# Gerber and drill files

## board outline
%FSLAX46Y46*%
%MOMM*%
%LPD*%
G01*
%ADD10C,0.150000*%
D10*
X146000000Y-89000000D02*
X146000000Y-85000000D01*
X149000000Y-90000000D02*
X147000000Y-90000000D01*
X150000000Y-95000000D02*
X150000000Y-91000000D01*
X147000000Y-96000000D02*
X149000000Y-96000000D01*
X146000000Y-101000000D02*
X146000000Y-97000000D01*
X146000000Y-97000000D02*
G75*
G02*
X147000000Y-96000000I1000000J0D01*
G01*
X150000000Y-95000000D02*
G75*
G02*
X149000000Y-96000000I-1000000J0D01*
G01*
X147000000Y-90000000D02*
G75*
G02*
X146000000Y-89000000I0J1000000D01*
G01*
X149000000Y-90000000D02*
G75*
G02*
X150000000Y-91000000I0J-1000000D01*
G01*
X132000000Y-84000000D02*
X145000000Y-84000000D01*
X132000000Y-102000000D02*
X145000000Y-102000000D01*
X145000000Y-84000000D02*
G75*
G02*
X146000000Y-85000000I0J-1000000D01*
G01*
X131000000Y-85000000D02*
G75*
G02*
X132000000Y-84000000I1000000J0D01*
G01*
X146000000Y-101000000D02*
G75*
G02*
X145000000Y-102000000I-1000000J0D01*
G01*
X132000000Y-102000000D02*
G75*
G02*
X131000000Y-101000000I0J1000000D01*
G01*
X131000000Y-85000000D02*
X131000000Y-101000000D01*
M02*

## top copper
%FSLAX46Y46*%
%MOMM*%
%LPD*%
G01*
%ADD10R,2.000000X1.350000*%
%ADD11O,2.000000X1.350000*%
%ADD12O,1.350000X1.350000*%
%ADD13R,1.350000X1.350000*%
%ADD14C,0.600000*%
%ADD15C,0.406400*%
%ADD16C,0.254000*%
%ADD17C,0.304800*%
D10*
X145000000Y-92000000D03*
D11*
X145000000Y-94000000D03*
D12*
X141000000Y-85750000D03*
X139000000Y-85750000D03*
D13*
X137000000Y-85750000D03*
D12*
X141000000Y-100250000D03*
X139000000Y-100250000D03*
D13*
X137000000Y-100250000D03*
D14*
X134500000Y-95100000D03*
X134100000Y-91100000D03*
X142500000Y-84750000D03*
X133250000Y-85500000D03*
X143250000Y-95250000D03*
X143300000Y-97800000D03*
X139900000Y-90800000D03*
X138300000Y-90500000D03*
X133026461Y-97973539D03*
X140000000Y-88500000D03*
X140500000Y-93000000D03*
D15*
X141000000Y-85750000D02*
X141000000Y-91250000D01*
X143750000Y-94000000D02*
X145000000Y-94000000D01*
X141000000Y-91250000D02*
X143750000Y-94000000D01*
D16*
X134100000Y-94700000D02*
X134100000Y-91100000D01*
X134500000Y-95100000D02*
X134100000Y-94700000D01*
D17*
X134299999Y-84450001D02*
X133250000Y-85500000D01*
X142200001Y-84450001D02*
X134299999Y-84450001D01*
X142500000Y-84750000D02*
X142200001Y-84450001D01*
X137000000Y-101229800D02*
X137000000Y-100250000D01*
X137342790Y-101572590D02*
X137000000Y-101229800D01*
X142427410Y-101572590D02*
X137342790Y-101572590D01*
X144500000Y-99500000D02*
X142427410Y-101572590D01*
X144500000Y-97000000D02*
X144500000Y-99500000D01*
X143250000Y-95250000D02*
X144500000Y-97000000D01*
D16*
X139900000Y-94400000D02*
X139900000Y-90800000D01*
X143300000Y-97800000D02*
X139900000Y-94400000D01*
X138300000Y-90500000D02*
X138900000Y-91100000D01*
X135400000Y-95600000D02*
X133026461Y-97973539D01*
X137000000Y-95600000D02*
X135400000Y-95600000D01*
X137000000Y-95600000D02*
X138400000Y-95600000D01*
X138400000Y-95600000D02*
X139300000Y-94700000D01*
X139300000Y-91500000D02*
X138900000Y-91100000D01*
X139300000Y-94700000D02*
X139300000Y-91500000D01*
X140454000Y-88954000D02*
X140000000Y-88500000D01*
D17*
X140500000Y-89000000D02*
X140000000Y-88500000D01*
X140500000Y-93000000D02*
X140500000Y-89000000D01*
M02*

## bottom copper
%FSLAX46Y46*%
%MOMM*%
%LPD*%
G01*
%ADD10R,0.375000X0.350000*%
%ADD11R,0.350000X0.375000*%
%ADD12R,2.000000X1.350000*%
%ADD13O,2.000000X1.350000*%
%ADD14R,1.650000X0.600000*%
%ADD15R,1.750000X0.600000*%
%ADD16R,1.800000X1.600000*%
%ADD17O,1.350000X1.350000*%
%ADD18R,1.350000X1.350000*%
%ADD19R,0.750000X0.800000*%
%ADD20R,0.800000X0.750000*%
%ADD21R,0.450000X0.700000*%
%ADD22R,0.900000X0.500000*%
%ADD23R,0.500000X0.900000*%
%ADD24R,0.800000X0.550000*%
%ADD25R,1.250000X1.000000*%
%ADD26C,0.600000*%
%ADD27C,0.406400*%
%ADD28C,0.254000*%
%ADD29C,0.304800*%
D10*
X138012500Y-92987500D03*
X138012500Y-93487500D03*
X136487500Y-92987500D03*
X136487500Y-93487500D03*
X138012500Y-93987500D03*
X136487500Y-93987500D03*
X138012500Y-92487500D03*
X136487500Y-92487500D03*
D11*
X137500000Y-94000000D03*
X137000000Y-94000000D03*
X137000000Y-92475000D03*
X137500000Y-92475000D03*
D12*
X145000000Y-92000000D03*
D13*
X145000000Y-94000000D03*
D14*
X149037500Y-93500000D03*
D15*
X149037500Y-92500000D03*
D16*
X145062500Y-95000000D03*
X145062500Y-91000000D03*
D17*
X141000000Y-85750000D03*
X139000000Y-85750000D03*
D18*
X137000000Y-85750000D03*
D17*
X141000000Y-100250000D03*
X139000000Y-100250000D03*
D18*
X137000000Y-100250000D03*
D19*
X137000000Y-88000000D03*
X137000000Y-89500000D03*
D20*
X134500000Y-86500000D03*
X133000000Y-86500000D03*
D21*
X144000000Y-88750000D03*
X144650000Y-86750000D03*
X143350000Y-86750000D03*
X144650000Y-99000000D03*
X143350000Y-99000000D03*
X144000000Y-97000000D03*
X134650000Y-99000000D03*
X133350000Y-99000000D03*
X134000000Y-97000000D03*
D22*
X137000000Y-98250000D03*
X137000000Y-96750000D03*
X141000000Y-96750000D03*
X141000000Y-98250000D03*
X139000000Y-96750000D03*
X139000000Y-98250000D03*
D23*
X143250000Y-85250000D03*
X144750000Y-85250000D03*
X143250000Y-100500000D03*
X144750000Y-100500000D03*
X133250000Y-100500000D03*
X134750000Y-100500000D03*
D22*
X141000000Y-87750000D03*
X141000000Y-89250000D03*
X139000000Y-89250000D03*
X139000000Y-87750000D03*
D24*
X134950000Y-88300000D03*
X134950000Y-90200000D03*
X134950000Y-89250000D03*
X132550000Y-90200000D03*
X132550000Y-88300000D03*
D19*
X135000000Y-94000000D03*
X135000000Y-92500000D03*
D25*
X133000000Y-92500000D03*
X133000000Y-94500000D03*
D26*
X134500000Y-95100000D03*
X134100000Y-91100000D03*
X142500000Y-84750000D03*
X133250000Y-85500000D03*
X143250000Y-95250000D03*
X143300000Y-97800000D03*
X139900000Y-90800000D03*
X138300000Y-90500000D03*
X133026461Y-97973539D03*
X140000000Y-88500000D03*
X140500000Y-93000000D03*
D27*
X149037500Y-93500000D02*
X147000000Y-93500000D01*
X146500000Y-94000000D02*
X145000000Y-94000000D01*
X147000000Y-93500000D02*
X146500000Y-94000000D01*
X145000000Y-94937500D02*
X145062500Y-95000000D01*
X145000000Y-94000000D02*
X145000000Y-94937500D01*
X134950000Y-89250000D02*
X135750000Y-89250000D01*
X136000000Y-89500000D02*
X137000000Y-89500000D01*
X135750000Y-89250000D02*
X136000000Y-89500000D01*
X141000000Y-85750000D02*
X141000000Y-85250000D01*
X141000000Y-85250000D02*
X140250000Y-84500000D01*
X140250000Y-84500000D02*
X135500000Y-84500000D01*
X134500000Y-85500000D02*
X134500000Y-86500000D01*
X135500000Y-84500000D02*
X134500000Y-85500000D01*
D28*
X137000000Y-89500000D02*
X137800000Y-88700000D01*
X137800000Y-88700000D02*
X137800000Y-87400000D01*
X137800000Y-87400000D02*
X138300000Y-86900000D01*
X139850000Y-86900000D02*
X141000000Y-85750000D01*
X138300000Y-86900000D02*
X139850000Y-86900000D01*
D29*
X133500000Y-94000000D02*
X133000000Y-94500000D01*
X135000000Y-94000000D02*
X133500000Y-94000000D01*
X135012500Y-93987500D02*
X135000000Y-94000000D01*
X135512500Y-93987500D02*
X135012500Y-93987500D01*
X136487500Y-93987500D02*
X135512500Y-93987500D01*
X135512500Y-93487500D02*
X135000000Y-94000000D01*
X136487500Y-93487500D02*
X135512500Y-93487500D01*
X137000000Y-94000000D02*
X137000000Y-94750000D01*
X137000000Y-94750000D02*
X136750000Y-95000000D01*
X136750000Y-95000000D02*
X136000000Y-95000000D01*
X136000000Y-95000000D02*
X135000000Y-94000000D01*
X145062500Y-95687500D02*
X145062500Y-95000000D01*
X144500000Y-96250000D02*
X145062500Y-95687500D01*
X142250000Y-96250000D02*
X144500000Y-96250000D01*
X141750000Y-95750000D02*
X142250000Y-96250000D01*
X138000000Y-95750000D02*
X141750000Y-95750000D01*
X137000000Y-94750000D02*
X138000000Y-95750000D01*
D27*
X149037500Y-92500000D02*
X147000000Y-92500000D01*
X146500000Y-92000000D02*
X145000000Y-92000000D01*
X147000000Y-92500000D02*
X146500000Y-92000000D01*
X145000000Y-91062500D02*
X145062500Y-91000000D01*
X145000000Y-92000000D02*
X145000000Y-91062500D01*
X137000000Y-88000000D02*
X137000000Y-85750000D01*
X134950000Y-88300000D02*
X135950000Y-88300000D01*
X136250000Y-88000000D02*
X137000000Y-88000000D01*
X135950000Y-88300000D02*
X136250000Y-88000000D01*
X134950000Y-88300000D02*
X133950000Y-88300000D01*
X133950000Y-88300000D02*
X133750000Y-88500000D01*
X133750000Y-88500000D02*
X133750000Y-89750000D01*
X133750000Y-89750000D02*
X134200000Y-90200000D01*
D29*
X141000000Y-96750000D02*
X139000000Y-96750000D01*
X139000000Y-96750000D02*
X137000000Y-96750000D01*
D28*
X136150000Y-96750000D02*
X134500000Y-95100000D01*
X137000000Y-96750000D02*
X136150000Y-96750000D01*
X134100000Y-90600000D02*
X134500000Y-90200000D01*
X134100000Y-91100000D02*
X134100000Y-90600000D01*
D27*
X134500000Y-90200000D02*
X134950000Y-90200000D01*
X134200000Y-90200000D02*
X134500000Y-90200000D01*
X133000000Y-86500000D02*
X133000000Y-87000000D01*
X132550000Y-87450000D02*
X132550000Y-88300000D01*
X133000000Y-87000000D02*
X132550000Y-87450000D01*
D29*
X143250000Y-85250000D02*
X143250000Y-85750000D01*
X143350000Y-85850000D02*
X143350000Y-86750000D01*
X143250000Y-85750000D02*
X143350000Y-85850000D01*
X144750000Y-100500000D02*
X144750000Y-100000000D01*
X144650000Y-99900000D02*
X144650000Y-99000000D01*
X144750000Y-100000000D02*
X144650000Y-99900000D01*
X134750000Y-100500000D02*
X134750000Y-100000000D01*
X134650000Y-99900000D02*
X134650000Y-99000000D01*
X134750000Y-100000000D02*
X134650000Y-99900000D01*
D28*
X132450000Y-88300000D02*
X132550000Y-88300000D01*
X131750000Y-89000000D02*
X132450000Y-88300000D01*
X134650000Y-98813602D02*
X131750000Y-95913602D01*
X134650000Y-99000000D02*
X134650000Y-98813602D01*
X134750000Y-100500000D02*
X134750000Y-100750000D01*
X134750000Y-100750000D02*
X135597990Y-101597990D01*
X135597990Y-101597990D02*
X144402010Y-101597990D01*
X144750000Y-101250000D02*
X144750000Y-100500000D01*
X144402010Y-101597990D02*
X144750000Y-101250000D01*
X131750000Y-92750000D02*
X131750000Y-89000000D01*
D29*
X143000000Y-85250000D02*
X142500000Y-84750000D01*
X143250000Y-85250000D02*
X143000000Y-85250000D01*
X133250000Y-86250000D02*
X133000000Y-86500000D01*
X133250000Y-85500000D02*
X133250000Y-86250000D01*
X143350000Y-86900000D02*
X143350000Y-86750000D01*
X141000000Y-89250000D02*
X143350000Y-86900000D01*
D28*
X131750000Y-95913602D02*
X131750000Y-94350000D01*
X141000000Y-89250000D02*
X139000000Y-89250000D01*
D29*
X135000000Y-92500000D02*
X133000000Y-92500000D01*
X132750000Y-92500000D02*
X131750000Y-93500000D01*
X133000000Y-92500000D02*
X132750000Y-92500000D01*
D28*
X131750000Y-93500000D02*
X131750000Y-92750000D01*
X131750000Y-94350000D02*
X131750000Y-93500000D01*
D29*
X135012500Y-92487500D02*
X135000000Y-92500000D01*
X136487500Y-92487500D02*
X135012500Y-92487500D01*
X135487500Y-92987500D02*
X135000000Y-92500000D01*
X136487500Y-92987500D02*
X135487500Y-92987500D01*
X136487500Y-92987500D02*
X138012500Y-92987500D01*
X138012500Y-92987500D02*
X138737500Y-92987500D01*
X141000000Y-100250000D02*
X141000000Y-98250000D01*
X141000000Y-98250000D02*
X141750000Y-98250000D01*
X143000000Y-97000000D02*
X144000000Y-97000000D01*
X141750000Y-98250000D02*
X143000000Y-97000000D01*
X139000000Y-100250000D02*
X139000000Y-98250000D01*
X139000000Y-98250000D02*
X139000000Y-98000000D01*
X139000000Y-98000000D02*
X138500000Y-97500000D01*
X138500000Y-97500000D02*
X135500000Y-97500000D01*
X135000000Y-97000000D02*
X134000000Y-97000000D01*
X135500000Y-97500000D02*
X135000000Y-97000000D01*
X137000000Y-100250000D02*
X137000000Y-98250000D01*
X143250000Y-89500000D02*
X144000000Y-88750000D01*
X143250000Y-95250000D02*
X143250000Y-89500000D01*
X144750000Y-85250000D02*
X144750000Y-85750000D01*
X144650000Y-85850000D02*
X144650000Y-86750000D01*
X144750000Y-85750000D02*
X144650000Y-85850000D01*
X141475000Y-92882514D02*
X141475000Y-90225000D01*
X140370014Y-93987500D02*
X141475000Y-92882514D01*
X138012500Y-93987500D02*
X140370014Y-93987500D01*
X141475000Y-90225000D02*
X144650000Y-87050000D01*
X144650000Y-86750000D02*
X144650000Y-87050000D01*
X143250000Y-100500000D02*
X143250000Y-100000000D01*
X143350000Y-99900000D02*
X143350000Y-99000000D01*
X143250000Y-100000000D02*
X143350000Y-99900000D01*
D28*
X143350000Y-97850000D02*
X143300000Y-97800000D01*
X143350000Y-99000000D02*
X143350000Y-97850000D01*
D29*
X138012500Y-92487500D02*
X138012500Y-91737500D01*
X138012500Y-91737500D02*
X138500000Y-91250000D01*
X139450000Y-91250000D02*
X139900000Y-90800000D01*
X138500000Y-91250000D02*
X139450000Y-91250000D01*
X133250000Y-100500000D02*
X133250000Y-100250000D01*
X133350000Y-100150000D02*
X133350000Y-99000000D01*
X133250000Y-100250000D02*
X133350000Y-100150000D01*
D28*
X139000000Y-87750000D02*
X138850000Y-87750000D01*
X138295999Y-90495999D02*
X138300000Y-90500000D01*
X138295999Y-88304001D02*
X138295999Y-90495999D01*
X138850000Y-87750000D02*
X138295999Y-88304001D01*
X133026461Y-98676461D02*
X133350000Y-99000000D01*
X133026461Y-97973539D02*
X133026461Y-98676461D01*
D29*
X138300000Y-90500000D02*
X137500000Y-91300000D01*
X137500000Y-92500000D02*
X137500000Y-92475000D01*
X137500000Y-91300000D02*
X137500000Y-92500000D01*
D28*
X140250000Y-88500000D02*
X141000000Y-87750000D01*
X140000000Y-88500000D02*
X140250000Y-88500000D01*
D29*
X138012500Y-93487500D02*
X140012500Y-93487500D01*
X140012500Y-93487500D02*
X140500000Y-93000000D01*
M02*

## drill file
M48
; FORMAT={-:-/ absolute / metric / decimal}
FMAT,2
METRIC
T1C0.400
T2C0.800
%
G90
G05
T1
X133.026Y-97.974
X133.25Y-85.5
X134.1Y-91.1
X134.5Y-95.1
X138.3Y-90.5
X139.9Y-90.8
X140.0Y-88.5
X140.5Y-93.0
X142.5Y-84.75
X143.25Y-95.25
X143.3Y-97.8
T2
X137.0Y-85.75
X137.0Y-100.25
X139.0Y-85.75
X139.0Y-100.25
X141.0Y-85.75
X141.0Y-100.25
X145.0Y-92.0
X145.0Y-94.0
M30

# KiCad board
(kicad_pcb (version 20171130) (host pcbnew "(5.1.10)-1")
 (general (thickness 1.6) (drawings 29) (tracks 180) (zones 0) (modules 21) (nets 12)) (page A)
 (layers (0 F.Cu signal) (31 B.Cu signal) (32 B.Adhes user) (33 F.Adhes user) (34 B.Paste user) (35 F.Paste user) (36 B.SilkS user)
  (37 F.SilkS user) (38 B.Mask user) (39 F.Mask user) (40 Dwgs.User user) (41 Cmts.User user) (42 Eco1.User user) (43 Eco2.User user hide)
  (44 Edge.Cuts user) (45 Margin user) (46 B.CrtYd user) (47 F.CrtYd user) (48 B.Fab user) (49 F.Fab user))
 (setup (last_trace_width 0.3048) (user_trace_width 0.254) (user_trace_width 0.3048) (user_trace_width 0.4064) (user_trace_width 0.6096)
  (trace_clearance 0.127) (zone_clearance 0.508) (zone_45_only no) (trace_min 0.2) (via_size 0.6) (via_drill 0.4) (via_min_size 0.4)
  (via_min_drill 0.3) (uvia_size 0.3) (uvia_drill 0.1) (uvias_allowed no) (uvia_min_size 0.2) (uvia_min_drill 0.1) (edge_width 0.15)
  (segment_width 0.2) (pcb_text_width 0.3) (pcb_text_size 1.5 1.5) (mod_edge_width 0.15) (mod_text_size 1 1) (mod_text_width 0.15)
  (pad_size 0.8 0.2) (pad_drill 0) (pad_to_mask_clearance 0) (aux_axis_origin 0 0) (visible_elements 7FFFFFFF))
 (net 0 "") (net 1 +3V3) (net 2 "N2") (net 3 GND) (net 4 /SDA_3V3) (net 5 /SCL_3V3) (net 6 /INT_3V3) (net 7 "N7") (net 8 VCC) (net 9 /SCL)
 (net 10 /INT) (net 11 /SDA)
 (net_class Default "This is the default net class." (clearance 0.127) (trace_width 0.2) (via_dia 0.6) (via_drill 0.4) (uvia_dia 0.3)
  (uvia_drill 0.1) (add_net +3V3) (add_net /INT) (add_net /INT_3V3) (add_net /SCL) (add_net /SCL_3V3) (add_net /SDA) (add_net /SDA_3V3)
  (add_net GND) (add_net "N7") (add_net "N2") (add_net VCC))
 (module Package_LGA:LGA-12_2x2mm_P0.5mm (layer B.Cu) (at 137.25 93.2375 180)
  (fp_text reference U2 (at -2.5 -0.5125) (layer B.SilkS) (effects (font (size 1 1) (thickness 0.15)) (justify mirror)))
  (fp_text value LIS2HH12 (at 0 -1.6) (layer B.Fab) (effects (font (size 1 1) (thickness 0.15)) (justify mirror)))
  (pad 2 smd rect (at -0.7625 0.25 180) (size 0.375 0.35) (layers B.Cu B.Paste B.Mask) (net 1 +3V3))
  (pad 3 smd rect (at -0.7625 -0.25 180) (size 0.375 0.35) (layers B.Cu B.Paste B.Mask) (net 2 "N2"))
  (pad 9 smd rect (at 0.7625 0.25 180) (size 0.375 0.35) (layers B.Cu B.Paste B.Mask) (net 1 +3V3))
  (pad 8 smd rect (at 0.7625 -0.25 180) (size 0.375 0.35) (layers B.Cu B.Paste B.Mask) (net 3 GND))
  (pad 4 smd rect (at -0.7625 -0.75 180) (size 0.375 0.35) (layers B.Cu B.Paste B.Mask) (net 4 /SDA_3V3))
  (pad 7 smd rect (at 0.7625 -0.75 180) (size 0.375 0.35) (layers B.Cu B.Paste B.Mask) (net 3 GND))
  (pad 1 smd rect (at -0.7625 0.75 180) (size 0.375 0.35) (layers B.Cu B.Paste B.Mask) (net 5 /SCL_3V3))
  (pad 10 smd rect (at 0.7625 0.75 180) (size 0.375 0.35) (layers B.Cu B.Paste B.Mask) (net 1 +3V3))
  (pad 5 smd rect (at -0.25 -0.7625 90) (size 0.375 0.35) (layers B.Cu B.Paste B.Mask))
  (pad 6 smd rect (at 0.25 -0.7625 90) (size 0.375 0.35) (layers B.Cu B.Paste B.Mask) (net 3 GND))
  (pad 11 smd rect (at 0.25 0.7625 90) (size 0.375 0.35) (layers B.Cu B.Paste B.Mask))
  (pad 12 smd rect (at -0.25 0.7625 90) (size 0.375 0.35) (layers B.Cu B.Paste B.Mask) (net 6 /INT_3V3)))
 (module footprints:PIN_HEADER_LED (layer B.Cu) (at 145 92 180)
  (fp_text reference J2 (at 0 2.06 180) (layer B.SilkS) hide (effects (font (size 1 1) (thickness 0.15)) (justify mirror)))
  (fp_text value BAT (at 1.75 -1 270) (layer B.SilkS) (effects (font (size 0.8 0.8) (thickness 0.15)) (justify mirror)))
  (pad 1 thru_hole rect (at 0 0 180) (size 2 1.35) (drill 0.8) (layers *.Cu *.Mask) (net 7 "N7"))
  (pad 2 thru_hole oval (at 0 -2 180) (size 2 1.35) (drill 0.8) (layers *.Cu *.Mask) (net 3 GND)))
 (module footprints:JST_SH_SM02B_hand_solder (layer B.Cu) (at 147 93 90)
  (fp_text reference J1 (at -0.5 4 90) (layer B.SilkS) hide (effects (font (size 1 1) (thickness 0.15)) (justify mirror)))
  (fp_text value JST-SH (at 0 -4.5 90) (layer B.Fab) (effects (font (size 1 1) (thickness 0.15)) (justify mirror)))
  (pad 1 smd rect (at -0.5 2.0375 90) (size 0.6 1.65) (layers B.Cu B.Paste B.Mask) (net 3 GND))
  (pad 2 smd rect (at 0.5 2.0375 90) (size 0.6 1.75) (layers B.Cu B.Paste B.Mask) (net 7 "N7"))
  (pad 1 smd rect (at -2 -1.9375 90) (size 1.6 1.8) (layers B.Cu B.Paste B.Mask) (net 3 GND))
  (pad 2 smd rect (at 2 -1.9375 90) (size 1.6 1.8) (layers B.Cu B.Paste B.Mask) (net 7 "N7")))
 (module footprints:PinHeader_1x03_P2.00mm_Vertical (layer B.Cu) (at 137 85.75 270)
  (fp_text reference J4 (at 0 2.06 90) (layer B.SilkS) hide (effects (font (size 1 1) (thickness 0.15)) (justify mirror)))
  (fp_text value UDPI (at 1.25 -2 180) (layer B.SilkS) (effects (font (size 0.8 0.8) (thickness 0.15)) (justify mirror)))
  (pad 3 thru_hole oval (at 0 -4 270) (size 1.35 1.35) (drill 0.8) (layers *.Cu *.Mask) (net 3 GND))
  (pad 2 thru_hole oval (at 0 -2 270) (size 1.35 1.35) (drill 0.8) (layers *.Cu *.Mask))
  (pad 1 thru_hole rect (at 0 0 270) (size 1.35 1.35) (drill 0.8) (layers *.Cu *.Mask) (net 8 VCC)))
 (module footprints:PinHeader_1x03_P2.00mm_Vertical (layer B.Cu) (at 137 100.25 270)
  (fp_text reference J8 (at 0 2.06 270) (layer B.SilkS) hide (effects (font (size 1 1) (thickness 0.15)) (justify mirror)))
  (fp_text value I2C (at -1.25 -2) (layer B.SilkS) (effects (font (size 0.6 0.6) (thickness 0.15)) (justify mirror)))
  (pad 3 thru_hole oval (at 0 -4 270) (size 1.35 1.35) (drill 0.8) (layers *.Cu *.Mask) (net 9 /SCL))
  (pad 2 thru_hole oval (at 0 -2 270) (size 1.35 1.35) (drill 0.8) (layers *.Cu *.Mask) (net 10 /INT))
  (pad 1 thru_hole rect (at 0 0 270) (size 1.35 1.35) (drill 0.8) (layers *.Cu *.Mask) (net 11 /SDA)))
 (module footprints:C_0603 (layer B.Cu) (at 137 88.75 270)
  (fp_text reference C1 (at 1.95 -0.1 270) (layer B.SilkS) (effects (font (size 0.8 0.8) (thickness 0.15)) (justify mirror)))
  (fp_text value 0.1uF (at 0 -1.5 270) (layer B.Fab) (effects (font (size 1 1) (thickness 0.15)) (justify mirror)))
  (pad 1 smd rect (at -0.75 0 270) (size 0.8 0.75) (layers B.Cu B.Paste B.Mask) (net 8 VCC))
  (pad 2 smd rect (at 0.75 0 270) (size 0.8 0.75) (layers B.Cu B.Paste B.Mask) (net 3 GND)))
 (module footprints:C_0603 (layer B.Cu) (at 133.75 86.5)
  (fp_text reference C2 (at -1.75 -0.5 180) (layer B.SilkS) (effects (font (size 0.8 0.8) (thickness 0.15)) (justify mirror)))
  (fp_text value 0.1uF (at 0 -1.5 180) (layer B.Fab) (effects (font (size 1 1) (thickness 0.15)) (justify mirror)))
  (pad 2 smd rect (at 0.75 0) (size 0.8 0.75) (layers B.Cu B.Paste B.Mask) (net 3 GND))
  (pad 1 smd rect (at -0.75 0) (size 0.8 0.75) (layers B.Cu B.Paste B.Mask) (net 1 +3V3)))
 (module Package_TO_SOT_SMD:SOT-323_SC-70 (layer B.Cu) (at 144 87.75 270)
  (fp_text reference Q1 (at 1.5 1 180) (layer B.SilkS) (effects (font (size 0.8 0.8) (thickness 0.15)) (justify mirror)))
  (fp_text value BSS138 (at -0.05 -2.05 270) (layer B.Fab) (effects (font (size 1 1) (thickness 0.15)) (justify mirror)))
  (pad 3 smd rect (at 1 0) (size 0.45 0.7) (layers B.Cu B.Paste B.Mask) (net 11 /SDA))
  (pad 2 smd rect (at -1 -0.65) (size 0.45 0.7) (layers B.Cu B.Paste B.Mask) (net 4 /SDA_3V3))
  (pad 1 smd rect (at -1 0.65) (size 0.45 0.7) (layers B.Cu B.Paste B.Mask) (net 1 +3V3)))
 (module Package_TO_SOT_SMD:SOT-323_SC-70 (layer B.Cu) (at 144 98 90)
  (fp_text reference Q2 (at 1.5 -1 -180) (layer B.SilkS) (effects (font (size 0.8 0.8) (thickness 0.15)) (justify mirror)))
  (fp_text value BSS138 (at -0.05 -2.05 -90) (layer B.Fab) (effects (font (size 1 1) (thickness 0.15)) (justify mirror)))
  (pad 1 smd rect (at -1 0.65 180) (size 0.45 0.7) (layers B.Cu B.Paste B.Mask) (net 1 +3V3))
  (pad 2 smd rect (at -1 -0.65 180) (size 0.45 0.7) (layers B.Cu B.Paste B.Mask) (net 5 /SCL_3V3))
  (pad 3 smd rect (at 1 0 180) (size 0.45 0.7) (layers B.Cu B.Paste B.Mask) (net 9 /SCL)))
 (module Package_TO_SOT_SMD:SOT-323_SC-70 (layer B.Cu) (at 134 98 90)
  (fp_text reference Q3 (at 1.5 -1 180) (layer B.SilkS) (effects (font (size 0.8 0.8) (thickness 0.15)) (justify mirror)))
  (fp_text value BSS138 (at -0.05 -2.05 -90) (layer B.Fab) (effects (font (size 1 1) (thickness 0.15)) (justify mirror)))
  (pad 1 smd rect (at -1 0.65 180) (size 0.45 0.7) (layers B.Cu B.Paste B.Mask) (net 1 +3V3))
  (pad 2 smd rect (at -1 -0.65 180) (size 0.45 0.7) (layers B.Cu B.Paste B.Mask) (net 6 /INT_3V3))
  (pad 3 smd rect (at 1 0 180) (size 0.45 0.7) (layers B.Cu B.Paste B.Mask) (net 10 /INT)))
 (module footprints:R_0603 (layer B.Cu) (at 137 97.5 270)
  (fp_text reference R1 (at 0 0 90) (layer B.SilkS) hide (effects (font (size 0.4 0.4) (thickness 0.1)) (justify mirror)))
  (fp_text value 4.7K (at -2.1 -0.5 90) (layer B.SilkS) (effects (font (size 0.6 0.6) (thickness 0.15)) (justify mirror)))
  (pad 2 smd rect (at 0.75 0 270) (size 0.5 0.9) (layers B.Cu B.Paste B.Mask) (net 11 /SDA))
  (pad 1 smd rect (at -0.75 0 270) (size 0.5 0.9) (layers B.Cu B.Paste B.Mask) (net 8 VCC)))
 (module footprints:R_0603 (layer B.Cu) (at 141 97.5 270)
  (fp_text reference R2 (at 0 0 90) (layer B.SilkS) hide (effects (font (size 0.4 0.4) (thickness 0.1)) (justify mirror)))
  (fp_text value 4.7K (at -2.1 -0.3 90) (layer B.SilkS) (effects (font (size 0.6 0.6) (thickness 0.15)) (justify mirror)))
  (pad 1 smd rect (at -0.75 0 270) (size 0.5 0.9) (layers B.Cu B.Paste B.Mask) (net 8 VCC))
  (pad 2 smd rect (at 0.75 0 270) (size 0.5 0.9) (layers B.Cu B.Paste B.Mask) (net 9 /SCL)))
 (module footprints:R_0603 (layer B.Cu) (at 139 97.5 270)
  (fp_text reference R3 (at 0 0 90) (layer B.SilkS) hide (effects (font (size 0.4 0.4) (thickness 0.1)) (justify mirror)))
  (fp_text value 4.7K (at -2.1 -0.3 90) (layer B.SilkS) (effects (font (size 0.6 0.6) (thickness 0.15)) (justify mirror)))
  (pad 1 smd rect (at -0.75 0 270) (size 0.5 0.9) (layers B.Cu B.Paste B.Mask) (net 8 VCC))
  (pad 2 smd rect (at 0.75 0 270) (size 0.5 0.9) (layers B.Cu B.Paste B.Mask) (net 10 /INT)))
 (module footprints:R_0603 (layer B.Cu) (at 144 85.25)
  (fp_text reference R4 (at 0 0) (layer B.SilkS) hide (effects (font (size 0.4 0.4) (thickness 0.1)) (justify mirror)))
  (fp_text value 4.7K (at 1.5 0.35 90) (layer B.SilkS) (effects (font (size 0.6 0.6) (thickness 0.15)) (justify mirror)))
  (pad 1 smd rect (at -0.75 0) (size 0.5 0.9) (layers B.Cu B.Paste B.Mask) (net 1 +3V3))
  (pad 2 smd rect (at 0.75 0) (size 0.5 0.9) (layers B.Cu B.Paste B.Mask) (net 4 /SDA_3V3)))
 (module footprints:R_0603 (layer B.Cu) (at 144 100.5 180)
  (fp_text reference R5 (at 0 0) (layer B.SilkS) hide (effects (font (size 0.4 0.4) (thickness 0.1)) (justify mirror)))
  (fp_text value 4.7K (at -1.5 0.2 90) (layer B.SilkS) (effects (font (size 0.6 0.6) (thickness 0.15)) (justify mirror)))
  (pad 2 smd rect (at 0.75 0 180) (size 0.5 0.9) (layers B.Cu B.Paste B.Mask) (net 5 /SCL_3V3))
  (pad 1 smd rect (at -0.75 0 180) (size 0.5 0.9) (layers B.Cu B.Paste B.Mask) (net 1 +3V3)))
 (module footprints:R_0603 (layer B.Cu) (at 134 100.5 180)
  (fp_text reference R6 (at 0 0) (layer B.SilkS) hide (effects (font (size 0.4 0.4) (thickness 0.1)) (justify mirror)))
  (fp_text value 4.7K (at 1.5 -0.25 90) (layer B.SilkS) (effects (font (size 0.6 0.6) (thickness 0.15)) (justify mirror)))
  (pad 2 smd rect (at 0.75 0 180) (size 0.5 0.9) (layers B.Cu B.Paste B.Mask) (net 6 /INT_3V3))
  (pad 1 smd rect (at -0.75 0 180) (size 0.5 0.9) (layers B.Cu B.Paste B.Mask) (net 1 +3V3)))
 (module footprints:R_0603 (layer B.Cu) (at 141 88.5 90)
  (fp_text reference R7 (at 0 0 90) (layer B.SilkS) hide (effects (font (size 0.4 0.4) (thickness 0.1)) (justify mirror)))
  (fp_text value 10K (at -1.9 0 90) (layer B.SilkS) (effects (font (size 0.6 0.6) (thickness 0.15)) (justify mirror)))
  (pad 2 smd rect (at 0.75 0 90) (size 0.5 0.9) (layers B.Cu B.Paste B.Mask) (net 2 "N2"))
  (pad 1 smd rect (at -0.75 0 90) (size 0.5 0.9) (layers B.Cu B.Paste B.Mask) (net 1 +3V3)))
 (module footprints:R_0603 (layer B.Cu) (at 139 88.5 90)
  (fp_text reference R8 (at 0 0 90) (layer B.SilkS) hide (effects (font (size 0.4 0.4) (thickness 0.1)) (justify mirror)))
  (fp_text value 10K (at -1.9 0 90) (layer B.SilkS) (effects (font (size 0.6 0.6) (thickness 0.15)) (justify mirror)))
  (pad 1 smd rect (at -0.75 0 90) (size 0.5 0.9) (layers B.Cu B.Paste B.Mask) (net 1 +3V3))
  (pad 2 smd rect (at 0.75 0 90) (size 0.5 0.9) (layers B.Cu B.Paste B.Mask) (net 6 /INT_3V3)))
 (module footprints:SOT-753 (layer B.Cu) (at 133.75 89.25 270) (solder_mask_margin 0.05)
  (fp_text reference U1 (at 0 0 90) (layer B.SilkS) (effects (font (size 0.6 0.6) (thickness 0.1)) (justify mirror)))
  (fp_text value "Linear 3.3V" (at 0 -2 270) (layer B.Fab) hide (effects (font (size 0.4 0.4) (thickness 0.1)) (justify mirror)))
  (pad 1 smd rect (at -0.95 -1.2 270) (size 0.55 0.8) (layers B.Cu B.Paste B.Mask) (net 8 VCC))
  (pad 3 smd rect (at 0.95 -1.2 270) (size 0.55 0.8) (layers B.Cu B.Paste B.Mask) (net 8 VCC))
  (pad 2 smd rect (at 0 -1.2 270) (size 0.55 0.8) (layers B.Cu B.Paste B.Mask) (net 3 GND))
  (pad 4 smd rect (at 0.95 1.2 270) (size 0.55 0.8) (layers B.Cu B.Paste B.Mask))
  (pad 5 smd rect (at -0.95 1.2 270) (size 0.55 0.8) (layers B.Cu B.Paste B.Mask) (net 1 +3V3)))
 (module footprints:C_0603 (layer B.Cu) (at 135 93.25 270)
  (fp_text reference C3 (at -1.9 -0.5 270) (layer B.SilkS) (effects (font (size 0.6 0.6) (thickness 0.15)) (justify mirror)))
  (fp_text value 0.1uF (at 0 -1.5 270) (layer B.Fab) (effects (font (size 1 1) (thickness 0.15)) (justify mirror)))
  (pad 2 smd rect (at 0.75 0 270) (size 0.8 0.75) (layers B.Cu B.Paste B.Mask) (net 3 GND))
  (pad 1 smd rect (at -0.75 0 270) (size 0.8 0.75) (layers B.Cu B.Paste B.Mask) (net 1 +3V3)))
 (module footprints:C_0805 (layer B.Cu) (at 133 93.5 270)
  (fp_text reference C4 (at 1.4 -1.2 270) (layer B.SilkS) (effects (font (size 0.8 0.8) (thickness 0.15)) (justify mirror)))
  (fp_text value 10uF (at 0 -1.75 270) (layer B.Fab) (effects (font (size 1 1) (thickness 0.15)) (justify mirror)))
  (pad 1 smd rect (at -1 0 270) (size 1 1.25) (layers B.Cu B.Paste B.Mask) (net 1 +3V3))
  (pad 2 smd rect (at 1 0 270) (size 1 1.25) (layers B.Cu B.Paste B.Mask) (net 3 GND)))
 (gr_line (start 146 89) (end 146 85) (layer Edge.Cuts) (width 0.15))
 (gr_line (start 149 90) (end 147 90) (layer Edge.Cuts) (width 0.15))
 (gr_line (start 150 95) (end 150 91) (layer Edge.Cuts) (width 0.15))
 (gr_line (start 147 96) (end 149 96) (layer Edge.Cuts) (width 0.15))
 (gr_line (start 146 101) (end 146 97) (layer Edge.Cuts) (width 0.15))
 (gr_arc (start 147 97) (end 147 96) (angle -90) (layer Edge.Cuts) (width 0.15))
 (gr_arc (start 149 95) (end 149 96) (angle -90) (layer Edge.Cuts) (width 0.15))
 (gr_arc (start 147 89) (end 146 89) (angle -90) (layer Edge.Cuts) (width 0.15))
 (gr_arc (start 149 91) (end 150 91) (angle -90) (layer Edge.Cuts) (width 0.15))
 (gr_line (start 132 84) (end 145 84) (layer Edge.Cuts) (width 0.15))
 (gr_line (start 132 102) (end 145 102) (layer Edge.Cuts) (width 0.15))
 (gr_arc (start 145 85) (end 145 84) (angle 90) (layer Edge.Cuts) (width 0.15))
 (gr_arc (start 132 85) (end 131 85) (angle 90) (layer Edge.Cuts) (width 0.15))
 (gr_arc (start 145 101) (end 146 101) (angle 90) (layer Edge.Cuts) (width 0.15))
 (gr_arc (start 132 101) (end 132 102) (angle 90) (layer Edge.Cuts) (width 0.15))
 (gr_line (start 131 85) (end 131 101) (angle 90) (layer Edge.Cuts) (width 0.15))
 (segment (start 149.0375 93.5) (end 147 93.5) (width 0.4064) (layer B.Cu) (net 3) (status 10))
 (segment (start 146.5 94) (end 145 94) (width 0.4064) (layer B.Cu) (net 3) (status 20))
 (segment (start 147 93.5) (end 146.5 94) (width 0.4064) (layer B.Cu) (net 3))
 (segment (start 145 94.9375) (end 145.0625 95) (width 0.4064) (layer B.Cu) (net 3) (status 30))
 (segment (start 145 94) (end 145 94.9375) (width 0.4064) (layer B.Cu) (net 3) (status 30))
 (segment (start 134.95 89.25) (end 135.75 89.25) (width 0.4064) (layer B.Cu) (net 3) (status 10))
 (segment (start 136 89.5) (end 137 89.5) (width 0.4064) (layer B.Cu) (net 3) (status 20))
 (segment (start 135.75 89.25) (end 136 89.5) (width 0.4064) (layer B.Cu) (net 3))
 (segment (start 141 85.75) (end 141 85.25) (width 0.4064) (layer B.Cu) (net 3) (status 30))
 (segment (start 141 85.25) (end 140.25 84.5) (width 0.4064) (layer B.Cu) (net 3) (status 10))
 (segment (start 140.25 84.5) (end 135.5 84.5) (width 0.4064) (layer B.Cu) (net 3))
 (segment (start 134.5 85.5) (end 134.5 86.5) (width 0.4064) (layer B.Cu) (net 3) (status 20))
 (segment (start 135.5 84.5) (end 134.5 85.5) (width 0.4064) (layer B.Cu) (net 3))
 (segment (start 141 85.75) (end 141 91.25) (width 0.4064) (layer F.Cu) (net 3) (status 10))
 (segment (start 143.75 94) (end 145 94) (width 0.4064) (layer F.Cu) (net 3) (status 20))
 (segment (start 141 91.25) (end 143.75 94) (width 0.4064) (layer F.Cu) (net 3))
 (segment (start 137 89.5) (end 137.8 88.7) (width 0.254) (layer B.Cu) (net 3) (status 10))
 (segment (start 137.8 88.7) (end 137.8 87.4) (width 0.254) (layer B.Cu) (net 3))
 (segment (start 137.8 87.4) (end 138.3 86.9) (width 0.254) (layer B.Cu) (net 3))
 (segment (start 139.85 86.9) (end 141 85.75) (width 0.254) (layer B.Cu) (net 3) (status 20))
 (segment (start 138.3 86.9) (end 139.85 86.9) (width 0.254) (layer B.Cu) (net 3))
 (segment (start 133.5 94) (end 133 94.5) (width 0.3048) (layer B.Cu) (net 3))
 (segment (start 135 94) (end 133.5 94) (width 0.3048) (layer B.Cu) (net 3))
 (segment (start 135.0125 93.9875) (end 135 94) (width 0.3048) (layer B.Cu) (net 3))
 (segment (start 135.5125 93.9875) (end 135.0125 93.9875) (width 0.3048) (layer B.Cu) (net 3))
 (segment (start 136.4875 93.9875) (end 135.5125 93.9875) (width 0.3048) (layer B.Cu) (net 3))
 (segment (start 135.5125 93.4875) (end 135 94) (width 0.3048) (layer B.Cu) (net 3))
 (segment (start 136.4875 93.4875) (end 135.5125 93.4875) (width 0.3048) (layer B.Cu) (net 3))
 (segment (start 137 94) (end 137 94.75) (width 0.3048) (layer B.Cu) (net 3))
 (segment (start 137 94.75) (end 136.75 95) (width 0.3048) (layer B.Cu) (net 3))
 (segment (start 136.75 95) (end 136 95) (width 0.3048) (layer B.Cu) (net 3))
 (segment (start 136 95) (end 135 94) (width 0.3048) (layer B.Cu) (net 3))
 (segment (start 145.0625 95.6875) (end 145.0625 95) (width 0.3048) (layer B.Cu) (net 3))
 (segment (start 144.5 96.25) (end 145.0625 95.6875) (width 0.3048) (layer B.Cu) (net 3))
 (segment (start 142.25 96.25) (end 144.5 96.25) (width 0.3048) (layer B.Cu) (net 3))
 (segment (start 141.75 95.75) (end 142.25 96.25) (width 0.3048) (layer B.Cu) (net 3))
 (segment (start 138 95.75) (end 141.75 95.75) (width 0.3048) (layer B.Cu) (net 3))
 (segment (start 137 94.75) (end 138 95.75) (width 0.3048) (layer B.Cu) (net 3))
 (segment (start 149.0375 92.5) (end 147 92.5) (width 0.4064) (layer B.Cu) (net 7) (status 10))
 (segment (start 146.5 92) (end 145 92) (width 0.4064) (layer B.Cu) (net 7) (status 20))
 (segment (start 147 92.5) (end 146.5 92) (width 0.4064) (layer B.Cu) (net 7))
 (segment (start 145 91.0625) (end 145.0625 91) (width 0.4064) (layer B.Cu) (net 7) (status 30))
 (segment (start 145 92) (end 145 91.0625) (width 0.4064) (layer B.Cu) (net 7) (status 30))
 (segment (start 137 88) (end 137 85.75) (width 0.4064) (layer B.Cu) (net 8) (status 30))
 (segment (start 134.95 88.3) (end 135.95 88.3) (width 0.4064) (layer B.Cu) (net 8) (status 10))
 (segment (start 136.25 88) (end 137 88) (width 0.4064) (layer B.Cu) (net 8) (status 20))
 (segment (start 135.95 88.3) (end 136.25 88) (width 0.4064) (layer B.Cu) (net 8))
 (segment (start 134.95 88.3) (end 133.95 88.3) (width 0.4064) (layer B.Cu) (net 8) (status 10))
 (segment (start 133.95 88.3) (end 133.75 88.5) (width 0.4064) (layer B.Cu) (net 8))
 (segment (start 133.75 88.5) (end 133.75 89.75) (width 0.4064) (layer B.Cu) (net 8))
 (segment (start 133.75 89.75) (end 134.2 90.2) (width 0.4064) (layer B.Cu) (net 8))
 (segment (start 141 96.75) (end 139 96.75) (width 0.3048) (layer B.Cu) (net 8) (status 30))
 (segment (start 139 96.75) (end 137 96.75) (width 0.3048) (layer B.Cu) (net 8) (status 30))
 (via (at 134.5 95.1) (size 0.6) (drill 0.4) (layers F.Cu B.Cu) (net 8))
 (segment (start 136.15 96.75) (end 134.5 95.1) (width 0.254) (layer B.Cu) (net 8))
 (segment (start 137 96.75) (end 136.15 96.75) (width 0.254) (layer B.Cu) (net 8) (status 10))
 (via (at 134.1 91.1) (size 0.6) (drill 0.4) (layers F.Cu B.Cu) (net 8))
 (segment (start 134.1 94.7) (end 134.1 91.1) (width 0.254) (layer F.Cu) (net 8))
 (segment (start 134.5 95.1) (end 134.1 94.7) (width 0.254) (layer F.Cu) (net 8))
 (segment (start 134.1 90.6) (end 134.5 90.2) (width 0.254) (layer B.Cu) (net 8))
 (segment (start 134.1 91.1) (end 134.1 90.6) (width 0.254) (layer B.Cu) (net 8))
 (segment (start 134.5 90.2) (end 134.95 90.2) (width 0.4064) (layer B.Cu) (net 8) (status 20))
 (segment (start 134.2 90.2) (end 134.5 90.2) (width 0.4064) (layer B.Cu) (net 8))
 (segment (start 133 86.5) (end 133 87) (width 0.4064) (layer B.Cu) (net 1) (status 10))
 (segment (start 132.55 87.45) (end 132.55 88.3) (width 0.4064) (layer B.Cu) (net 1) (status 20))
 (segment (start 133 87) (end 132.55 87.45) (width 0.4064) (layer B.Cu) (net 1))
 (segment (start 143.25 85.25) (end 143.25 85.75) (width 0.3048) (layer B.Cu) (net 1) (status 10))
 (segment (start 143.35 85.85) (end 143.35 86.75) (width 0.3048) (layer B.Cu) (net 1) (status 20))
 (segment (start 143.25 85.75) (end 143.35 85.85) (width 0.3048) (layer B.Cu) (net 1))
 (segment (start 144.75 100.5) (end 144.75 100) (width 0.3048) (layer B.Cu) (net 1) (status 10))
 (segment (start 144.65 99.9) (end 144.65 99) (width 0.3048) (layer B.Cu) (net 1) (status 20))
 (segment (start 144.75 100) (end 144.65 99.9) (width 0.3048) (layer B.Cu) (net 1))
 (segment (start 134.75 100.5) (end 134.75 100) (width 0.3048) (layer B.Cu) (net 1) (status 10))
 (segment (start 134.65 99.9) (end 134.65 99) (width 0.3048) (layer B.Cu) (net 1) (status 20))
 (segment (start 134.75 100) (end 134.65 99.9) (width 0.3048) (layer B.Cu) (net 1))
 (segment (start 132.45 88.3) (end 132.55 88.3) (width 0.254) (layer B.Cu) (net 1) (status 30))
 (segment (start 131.75 89) (end 132.45 88.3) (width 0.254) (layer B.Cu) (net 1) (status 20))
 (segment (start 134.65 98.813602) (end 131.75 95.913602) (width 0.254) (layer B.Cu) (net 1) (status 10))
 (segment (start 134.65 99) (end 134.65 98.813602) (width 0.254) (layer B.Cu) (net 1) (status 30))
 (segment (start 134.75 100.5) (end 134.75 100.75) (width 0.254) (layer B.Cu) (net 1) (status 30))
 (segment (start 134.75 100.75) (end 135.59799 101.59799) (width 0.254) (layer B.Cu) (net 1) (status 10))
 (segment (start 135.59799 101.59799) (end 144.40201 101.59799) (width 0.254) (layer B.Cu) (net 1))
 (segment (start 144.75 101.25) (end 144.75 100.5) (width 0.254) (layer B.Cu) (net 1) (status 20))
 (segment (start 144.40201 101.59799) (end 144.75 101.25) (width 0.254) (layer B.Cu) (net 1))
 (segment (start 131.75 92.75) (end 131.75 89) (width 0.254) (layer B.Cu) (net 1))
 (via (at 142.5 84.75) (size 0.6) (drill 0.4) (layers F.Cu B.Cu) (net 1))
 (segment (start 143 85.25) (end 142.5 84.75) (width 0.3048) (layer B.Cu) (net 1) (status 10))
 (segment (start 143.25 85.25) (end 143 85.25) (width 0.3048) (layer B.Cu) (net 1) (status 30))
 (via (at 133.25 85.5) (size 0.6) (drill 0.4) (layers F.Cu B.Cu) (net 1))
 (segment (start 134.299999 84.450001) (end 133.25 85.5) (width 0.3048) (layer F.Cu) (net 1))
 (segment (start 142.200001 84.450001) (end 134.299999 84.450001) (width 0.3048) (layer F.Cu) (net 1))
 (segment (start 142.5 84.75) (end 142.200001 84.450001) (width 0.3048) (layer F.Cu) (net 1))
 (segment (start 133.25 86.25) (end 133 86.5) (width 0.3048) (layer B.Cu) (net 1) (status 30))
 (segment (start 133.25 85.5) (end 133.25 86.25) (width 0.3048) (layer B.Cu) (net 1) (status 20))
 (segment (start 143.35 86.9) (end 143.35 86.75) (width 0.3048) (layer B.Cu) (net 1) (status 30))
 (segment (start 141 89.25) (end 143.35 86.9) (width 0.3048) (layer B.Cu) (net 1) (status 30))
 (segment (start 131.75 95.913602) (end 131.75 94.35) (width 0.254) (layer B.Cu) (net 1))
 (segment (start 141 89.25) (end 139 89.25) (width 0.254) (layer B.Cu) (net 1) (status 30))
 (segment (start 135 92.5) (end 133 92.5) (width 0.3048) (layer B.Cu) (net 1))
 (segment (start 132.75 92.5) (end 131.75 93.5) (width 0.3048) (layer B.Cu) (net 1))
 (segment (start 133 92.5) (end 132.75 92.5) (width 0.3048) (layer B.Cu) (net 1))
 (segment (start 131.75 93.5) (end 131.75 92.75) (width 0.254) (layer B.Cu) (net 1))
 (segment (start 131.75 94.35) (end 131.75 93.5) (width 0.254) (layer B.Cu) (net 1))
 (segment (start 135.0125 92.4875) (end 135 92.5) (width 0.3048) (layer B.Cu) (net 1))
 (segment (start 136.4875 92.4875) (end 135.0125 92.4875) (width 0.3048) (layer B.Cu) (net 1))
 (segment (start 135.4875 92.9875) (end 135 92.5) (width 0.3048) (layer B.Cu) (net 1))
 (segment (start 136.4875 92.9875) (end 135.4875 92.9875) (width 0.3048) (layer B.Cu) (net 1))
 (segment (start 136.4875 92.9875) (end 138.0125 92.9875) (width 0.3048) (layer B.Cu) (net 1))
 (segment (start 138.0125 92.9875) (end 138.7375 92.9875) (width 0.3048) (layer B.Cu) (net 1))
 (segment (start 141 100.25) (end 141 98.25) (width 0.3048) (layer B.Cu) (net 9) (status 30))
 (segment (start 141 98.25) (end 141.75 98.25) (width 0.3048) (layer B.Cu) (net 9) (status 10))
 (segment (start 143 97) (end 144 97) (width 0.3048) (layer B.Cu) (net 9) (status 20))
 (segment (start 141.75 98.25) (end 143 97) (width 0.3048) (layer B.Cu) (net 9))
 (segment (start 139 100.25) (end 139 98.25) (width 0.3048) (layer B.Cu) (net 10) (status 30))
 (segment (start 139 98.25) (end 139 98) (width 0.3048) (layer B.Cu) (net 10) (status 30))
 (segment (start 139 98) (end 138.5 97.5) (width 0.3048) (layer B.Cu) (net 10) (status 10))
 (segment (start 138.5 97.5) (end 135.5 97.5) (width 0.3048) (layer B.Cu) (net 10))
 (segment (start 135 97) (end 134 97) (width 0.3048) (layer B.Cu) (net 10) (status 20))
 (segment (start 135.5 97.5) (end 135 97) (width 0.3048) (layer B.Cu) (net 10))
 (segment (start 137 100.25) (end 137 98.25) (width 0.3048) (layer B.Cu) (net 11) (status 30))
 (segment (start 143.25 89.5) (end 144 88.75) (width 0.3048) (layer B.Cu) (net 11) (status 20))
 (segment (start 143.25 95.25) (end 143.25 89.5) (width 0.3048) (layer B.Cu) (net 11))
 (segment (start 137 101.2298) (end 137 100.25) (width 0.3048) (layer F.Cu) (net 11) (status 20))
 (segment (start 137.34279 101.57259) (end 137 101.2298) (width 0.3048) (layer F.Cu) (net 11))
 (segment (start 142.42741 101.57259) (end 137.34279 101.57259) (width 0.3048) (layer F.Cu) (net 11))
 (segment (start 144.5 99.5) (end 142.42741 101.57259) (width 0.3048) (layer F.Cu) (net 11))
 (segment (start 144.5 97) (end 144.5 99.5) (width 0.3048) (layer F.Cu) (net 11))
 (segment (start 143.25 95.25) (end 144.5 97) (width 0.3048) (layer F.Cu) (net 11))
 (via (at 143.25 95.25) (size 0.6) (drill 0.4) (layers F.Cu B.Cu) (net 11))
 (segment (start 144.75 85.25) (end 144.75 85.75) (width 0.3048) (layer B.Cu) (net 4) (status 10))
 (segment (start 144.65 85.85) (end 144.65 86.75) (width 0.3048) (layer B.Cu) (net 4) (status 20))
 (segment (start 144.75 85.75) (end 144.65 85.85) (width 0.3048) (layer B.Cu) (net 4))
 (segment (start 141.475 92.882514) (end 141.475 90.225) (width 0.3048) (layer B.Cu) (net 4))
 (segment (start 140.370014 93.9875) (end 141.475 92.882514) (width 0.3048) (layer B.Cu) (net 4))
 (segment (start 138.0125 93.9875) (end 140.370014 93.9875) (width 0.3048) (layer B.Cu) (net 4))
 (segment (start 141.475 90.225) (end 144.65 87.05) (width 0.3048) (layer B.Cu) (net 4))
 (segment (start 144.65 86.75) (end 144.65 87.05) (width 0.3048) (layer B.Cu) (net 4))
 (segment (start 143.25 100.5) (end 143.25 100) (width 0.3048) (layer B.Cu) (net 5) (status 10))
 (segment (start 143.35 99.9) (end 143.35 99) (width 0.3048) (layer B.Cu) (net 5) (status 20))
 (segment (start 143.25 100) (end 143.35 99.9) (width 0.3048) (layer B.Cu) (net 5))
 (via (at 143.3 97.8) (size 0.6) (drill 0.4) (layers F.Cu B.Cu) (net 5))
 (segment (start 143.35 97.85) (end 143.3 97.8) (width 0.254) (layer B.Cu) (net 5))
 (segment (start 143.35 99) (end 143.35 97.85) (width 0.254) (layer B.Cu) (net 5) (status 10))
 (segment (start 139.9 94.4) (end 139.9 90.8) (width 0.254) (layer F.Cu) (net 5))
 (via (at 139.9 90.8) (size 0.6) (drill 0.4) (layers F.Cu B.Cu) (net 5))
 (segment (start 143.3 97.8) (end 139.9 94.4) (width 0.254) (layer F.Cu) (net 5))
 (segment (start 138.0125 92.4875) (end 138.0125 91.7375) (width 0.3048) (layer B.Cu) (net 5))
 (segment (start 138.0125 91.7375) (end 138.5 91.25) (width 0.3048) (layer B.Cu) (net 5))
 (segment (start 139.45 91.25) (end 139.9 90.8) (width 0.3048) (layer B.Cu) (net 5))
 (segment (start 138.5 91.25) (end 139.45 91.25) (width 0.3048) (layer B.Cu) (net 5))
 (segment (start 133.25 100.5) (end 133.25 100.25) (width 0.3048) (layer B.Cu) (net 6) (status 30))
 (segment (start 133.35 100.15) (end 133.35 99) (width 0.3048) (layer B.Cu) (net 6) (status 30))
 (segment (start 133.25 100.25) (end 133.35 100.15) (width 0.3048) (layer B.Cu) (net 6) (status 30))
 (segment (start 139 87.75) (end 138.85 87.75) (width 0.254) (layer B.Cu) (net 6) (status 30))
 (via (at 138.3 90.5) (size 0.6) (drill 0.4) (layers F.Cu B.Cu) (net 6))
 (segment (start 138.295999 90.495999) (end 138.3 90.5) (width 0.254) (layer B.Cu) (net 6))
 (segment (start 138.295999 88.304001) (end 138.295999 90.495999) (width 0.254) (layer B.Cu) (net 6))
 (segment (start 138.85 87.75) (end 138.295999 88.304001) (width 0.254) (layer B.Cu) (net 6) (status 10))
 (segment (start 138.3 90.5) (end 138.9 91.1) (width 0.254) (layer F.Cu) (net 6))
 (via (at 133.026461 97.973539) (size 0.6) (drill 0.4) (layers F.Cu B.Cu) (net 6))
 (segment (start 135.4 95.6) (end 133.026461 97.973539) (width 0.254) (layer F.Cu) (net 6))
 (segment (start 137 95.6) (end 135.4 95.6) (width 0.254) (layer F.Cu) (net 6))
 (segment (start 133.026461 98.676461) (end 133.35 99) (width 0.254) (layer B.Cu) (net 6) (status 20))
 (segment (start 133.026461 97.973539) (end 133.026461 98.676461) (width 0.254) (layer B.Cu) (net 6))
 (segment (start 137 95.6) (end 138.4 95.6) (width 0.254) (layer F.Cu) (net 6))
 (segment (start 138.4 95.6) (end 139.3 94.7) (width 0.254) (layer F.Cu) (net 6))
 (segment (start 139.3 91.5) (end 138.9 91.1) (width 0.254) (layer F.Cu) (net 6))
 (segment (start 139.3 94.7) (end 139.3 91.5) (width 0.254) (layer F.Cu) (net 6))
 (segment (start 138.3 90.5) (end 137.5 91.3) (width 0.3048) (layer B.Cu) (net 6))
 (segment (start 137.5 92.5) (end 137.5 92.475) (width 0.3048) (layer B.Cu) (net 6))
 (segment (start 137.5 91.3) (end 137.5 92.5) (width 0.3048) (layer B.Cu) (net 6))
 (via (at 140 88.5) (size 0.6) (drill 0.4) (layers F.Cu B.Cu) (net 2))
 (segment (start 140.454 88.954) (end 140 88.5) (width 0.254) (layer F.Cu) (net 2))
 (segment (start 140.25 88.5) (end 141 87.75) (width 0.254) (layer B.Cu) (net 2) (status 20))
 (segment (start 140 88.5) (end 140.25 88.5) (width 0.254) (layer B.Cu) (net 2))
 (segment (start 138.0125 93.4875) (end 140.0125 93.4875) (width 0.3048) (layer B.Cu) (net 2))
 (via (at 140.5 93) (size 0.6) (drill 0.4) (layers F.Cu B.Cu) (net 2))
 (segment (start 140.0125 93.4875) (end 140.5 93) (width 0.3048) (layer B.Cu) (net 2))
 (segment (start 140.5 89) (end 140 88.5) (width 0.3048) (layer F.Cu) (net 2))
 (segment (start 140.5 93) (end 140.5 89) (width 0.3048) (layer F.Cu) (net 2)))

